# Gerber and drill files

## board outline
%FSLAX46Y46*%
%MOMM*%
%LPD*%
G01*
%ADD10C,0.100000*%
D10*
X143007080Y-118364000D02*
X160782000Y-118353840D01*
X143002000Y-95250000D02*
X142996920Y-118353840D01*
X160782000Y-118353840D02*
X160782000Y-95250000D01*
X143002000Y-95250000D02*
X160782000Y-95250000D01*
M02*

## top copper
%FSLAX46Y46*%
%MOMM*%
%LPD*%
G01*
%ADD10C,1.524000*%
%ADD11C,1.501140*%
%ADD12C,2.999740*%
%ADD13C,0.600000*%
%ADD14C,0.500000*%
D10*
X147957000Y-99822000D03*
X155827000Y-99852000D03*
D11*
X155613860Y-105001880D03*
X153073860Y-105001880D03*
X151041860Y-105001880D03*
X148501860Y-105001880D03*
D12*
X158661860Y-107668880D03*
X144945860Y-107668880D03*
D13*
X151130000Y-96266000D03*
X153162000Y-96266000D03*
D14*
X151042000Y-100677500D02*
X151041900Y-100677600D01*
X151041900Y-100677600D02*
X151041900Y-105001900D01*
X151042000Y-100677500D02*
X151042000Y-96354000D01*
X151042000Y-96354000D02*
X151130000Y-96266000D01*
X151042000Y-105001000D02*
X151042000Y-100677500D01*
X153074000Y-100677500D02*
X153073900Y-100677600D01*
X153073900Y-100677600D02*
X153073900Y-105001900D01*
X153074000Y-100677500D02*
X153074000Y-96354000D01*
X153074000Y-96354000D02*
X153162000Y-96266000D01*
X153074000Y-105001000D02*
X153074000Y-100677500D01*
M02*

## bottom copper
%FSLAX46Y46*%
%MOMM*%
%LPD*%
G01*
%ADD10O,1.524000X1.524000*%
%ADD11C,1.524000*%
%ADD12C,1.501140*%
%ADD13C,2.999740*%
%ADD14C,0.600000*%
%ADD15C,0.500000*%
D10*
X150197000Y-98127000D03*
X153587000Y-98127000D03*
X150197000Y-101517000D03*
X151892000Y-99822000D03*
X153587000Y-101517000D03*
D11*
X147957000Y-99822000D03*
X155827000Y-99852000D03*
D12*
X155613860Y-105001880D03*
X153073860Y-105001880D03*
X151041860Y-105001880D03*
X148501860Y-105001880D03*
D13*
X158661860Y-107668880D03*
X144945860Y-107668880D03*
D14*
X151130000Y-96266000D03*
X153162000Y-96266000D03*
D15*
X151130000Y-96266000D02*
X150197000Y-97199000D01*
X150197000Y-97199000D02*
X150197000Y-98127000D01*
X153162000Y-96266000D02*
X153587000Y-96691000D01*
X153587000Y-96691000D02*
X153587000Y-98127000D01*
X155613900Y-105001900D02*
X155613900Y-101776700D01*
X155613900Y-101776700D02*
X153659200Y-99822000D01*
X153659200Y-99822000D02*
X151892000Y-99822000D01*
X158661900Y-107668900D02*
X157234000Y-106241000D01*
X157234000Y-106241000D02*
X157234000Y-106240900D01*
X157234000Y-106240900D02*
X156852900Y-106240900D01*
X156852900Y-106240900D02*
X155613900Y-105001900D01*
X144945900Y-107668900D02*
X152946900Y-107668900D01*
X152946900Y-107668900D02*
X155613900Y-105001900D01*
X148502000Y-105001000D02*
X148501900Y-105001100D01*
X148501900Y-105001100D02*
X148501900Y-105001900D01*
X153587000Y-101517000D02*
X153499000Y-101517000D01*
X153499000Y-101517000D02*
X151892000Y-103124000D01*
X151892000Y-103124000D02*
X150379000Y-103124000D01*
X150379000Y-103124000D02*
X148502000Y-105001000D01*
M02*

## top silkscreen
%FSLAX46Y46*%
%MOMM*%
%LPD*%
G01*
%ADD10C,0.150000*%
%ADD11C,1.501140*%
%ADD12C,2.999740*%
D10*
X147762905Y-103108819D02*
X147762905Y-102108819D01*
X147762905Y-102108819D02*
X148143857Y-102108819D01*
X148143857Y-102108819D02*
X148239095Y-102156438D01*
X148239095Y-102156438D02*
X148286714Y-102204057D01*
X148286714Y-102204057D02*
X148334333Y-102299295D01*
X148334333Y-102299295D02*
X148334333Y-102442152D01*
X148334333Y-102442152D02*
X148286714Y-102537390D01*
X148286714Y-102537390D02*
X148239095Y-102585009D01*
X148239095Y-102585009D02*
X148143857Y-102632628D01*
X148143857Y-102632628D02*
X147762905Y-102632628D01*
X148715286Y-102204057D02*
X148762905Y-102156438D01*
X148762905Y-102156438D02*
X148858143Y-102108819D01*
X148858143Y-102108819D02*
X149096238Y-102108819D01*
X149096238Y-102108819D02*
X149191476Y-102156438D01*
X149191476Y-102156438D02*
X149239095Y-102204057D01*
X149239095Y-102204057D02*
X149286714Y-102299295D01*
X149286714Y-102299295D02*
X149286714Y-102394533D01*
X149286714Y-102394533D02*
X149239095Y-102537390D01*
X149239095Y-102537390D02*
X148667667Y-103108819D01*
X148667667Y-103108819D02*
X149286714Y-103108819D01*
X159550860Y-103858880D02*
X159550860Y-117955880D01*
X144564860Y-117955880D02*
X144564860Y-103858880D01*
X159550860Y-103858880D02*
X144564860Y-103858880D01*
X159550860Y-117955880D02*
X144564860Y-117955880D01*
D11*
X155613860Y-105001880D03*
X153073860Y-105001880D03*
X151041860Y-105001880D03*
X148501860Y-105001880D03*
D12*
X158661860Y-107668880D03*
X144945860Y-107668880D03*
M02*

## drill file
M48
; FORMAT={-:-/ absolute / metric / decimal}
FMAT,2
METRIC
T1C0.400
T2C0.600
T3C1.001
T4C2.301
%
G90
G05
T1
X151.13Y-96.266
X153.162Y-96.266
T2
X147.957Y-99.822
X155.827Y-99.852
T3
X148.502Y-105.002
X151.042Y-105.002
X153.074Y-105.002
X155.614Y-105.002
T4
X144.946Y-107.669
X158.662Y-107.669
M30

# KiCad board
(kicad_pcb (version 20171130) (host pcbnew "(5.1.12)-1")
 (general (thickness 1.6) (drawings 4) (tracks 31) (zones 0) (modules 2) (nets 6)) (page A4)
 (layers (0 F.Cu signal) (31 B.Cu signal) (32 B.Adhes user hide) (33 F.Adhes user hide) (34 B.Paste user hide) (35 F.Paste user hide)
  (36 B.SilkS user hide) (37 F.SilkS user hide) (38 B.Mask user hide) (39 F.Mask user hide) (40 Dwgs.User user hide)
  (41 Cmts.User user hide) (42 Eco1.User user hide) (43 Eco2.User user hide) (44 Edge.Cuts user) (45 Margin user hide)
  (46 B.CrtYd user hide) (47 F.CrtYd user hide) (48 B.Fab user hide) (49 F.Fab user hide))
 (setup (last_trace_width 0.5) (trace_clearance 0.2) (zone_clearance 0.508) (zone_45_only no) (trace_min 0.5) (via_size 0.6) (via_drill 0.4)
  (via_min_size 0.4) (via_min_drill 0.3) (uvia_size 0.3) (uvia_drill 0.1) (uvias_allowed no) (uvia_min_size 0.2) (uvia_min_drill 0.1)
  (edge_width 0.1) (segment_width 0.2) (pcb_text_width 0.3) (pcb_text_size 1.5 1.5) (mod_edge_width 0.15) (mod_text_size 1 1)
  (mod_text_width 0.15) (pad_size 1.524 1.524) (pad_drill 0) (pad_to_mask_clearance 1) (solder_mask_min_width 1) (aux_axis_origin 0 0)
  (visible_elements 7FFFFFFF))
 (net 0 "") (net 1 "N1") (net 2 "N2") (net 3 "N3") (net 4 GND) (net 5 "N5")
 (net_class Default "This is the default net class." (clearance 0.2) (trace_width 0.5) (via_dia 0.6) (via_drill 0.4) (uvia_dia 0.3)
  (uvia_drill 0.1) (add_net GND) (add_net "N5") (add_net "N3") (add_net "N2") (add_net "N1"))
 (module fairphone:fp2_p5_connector (layer B.Cu) (at 151.892 99.822)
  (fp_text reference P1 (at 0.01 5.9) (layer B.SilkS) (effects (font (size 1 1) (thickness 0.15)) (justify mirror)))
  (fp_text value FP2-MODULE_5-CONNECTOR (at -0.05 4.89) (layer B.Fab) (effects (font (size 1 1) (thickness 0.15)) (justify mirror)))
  (pad 5 smd oval (at -1.695 -1.695) (size 1.524 1.524) (layers B.Cu B.Paste B.Mask) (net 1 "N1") (solder_mask_margin 1))
  (pad 4 smd oval (at 1.695 -1.695) (size 1.524 1.524) (layers B.Cu B.Paste) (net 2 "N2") (solder_mask_margin 1))
  (pad 2 smd oval (at -1.695 1.695) (size 1.524 1.524) (layers B.Cu B.Paste B.Mask) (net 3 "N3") (solder_mask_margin 1))
  (pad 3 smd oval (at 0 0) (size 1.524 1.524) (layers B.Cu B.Paste B.Mask) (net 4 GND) (solder_mask_margin 1))
  (pad 1 smd oval (at 1.695 1.695) (size 1.524 1.524) (layers B.Cu B.Paste B.Mask) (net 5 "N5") (solder_mask_margin 1))
  (pad "" thru_hole circle (at -3.935 0) (size 1.524 1.524) (drill 0.6) (layers *.Cu *.Mask B.SilkS))
  (pad "" thru_hole circle (at 3.935 0.03) (size 1.524 1.524) (drill 0.6) (layers *.Cu *.Mask B.SilkS)))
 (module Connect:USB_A (layer F.Cu) (at 148.501 105.004)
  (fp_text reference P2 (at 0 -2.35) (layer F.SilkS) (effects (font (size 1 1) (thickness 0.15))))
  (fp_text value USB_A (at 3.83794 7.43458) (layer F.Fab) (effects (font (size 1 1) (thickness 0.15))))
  (fp_line (start 11.04986 -1.14512) (end 11.04986 12.95188) (layer F.SilkS) (width 0.15))
  (fp_line (start -3.93614 12.95188) (end -3.93614 -1.14512) (layer F.SilkS) (width 0.15))
  (fp_line (start 11.04986 -1.14512) (end -3.93614 -1.14512) (layer F.SilkS) (width 0.15))
  (fp_line (start 11.04986 12.95188) (end -3.93614 12.95188) (layer F.SilkS) (width 0.15))
  (pad 4 thru_hole circle (at 7.11286 -0.00212 270) (size 1.50114 1.50114) (drill 1.00076) (layers *.Cu *.Mask F.SilkS) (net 4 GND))
  (pad 3 thru_hole circle (at 4.57286 -0.00212 270) (size 1.50114 1.50114) (drill 1.00076) (layers *.Cu *.Mask F.SilkS) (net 2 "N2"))
  (pad 2 thru_hole circle (at 2.54086 -0.00212 270) (size 1.50114 1.50114) (drill 1.00076) (layers *.Cu *.Mask F.SilkS) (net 1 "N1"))
  (pad 1 thru_hole circle (at 0.00086 -0.00212 270) (size 1.50114 1.50114) (drill 1.00076) (layers *.Cu *.Mask F.SilkS) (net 5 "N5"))
  (pad 5 thru_hole circle (at 10.16086 2.66488 270) (size 2.99974 2.99974) (drill 2.30124) (layers *.Cu *.Mask F.SilkS) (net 4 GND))
  (pad 5 thru_hole circle (at -3.55514 2.66488 270) (size 2.99974 2.99974) (drill 2.30124) (layers *.Cu *.Mask F.SilkS) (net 4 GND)))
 (gr_line (start 143.00708 118.364) (end 160.782 118.35384) (layer Edge.Cuts) (width 0.1))
 (gr_line (start 143.002 95.25) (end 142.99692 118.35384) (angle 90) (layer Edge.Cuts) (width 0.1))
 (gr_line (start 160.782 118.35384) (end 160.782 95.25) (angle 90) (layer Edge.Cuts) (width 0.1))
 (gr_line (start 143.002 95.25) (end 160.782 95.25) (angle 90) (layer Edge.Cuts) (width 0.1))
 (segment (start 151.042 100.6775) (end 151.0419 100.6776) (width 0.5) (layer F.Cu) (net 1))
 (segment (start 151.0419 100.6776) (end 151.0419 105.0019) (width 0.5) (layer F.Cu) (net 1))
 (segment (start 151.042 100.6775) (end 151.042 96.354) (width 0.5) (layer F.Cu) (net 1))
 (segment (start 151.042 96.354) (end 151.13 96.266) (width 0.5) (layer F.Cu) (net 1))
 (segment (start 151.042 105.001) (end 151.042 100.6775) (width 0.5) (layer F.Cu) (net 1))
 (segment (start 151.13 96.266) (end 150.197 97.199) (width 0.5) (layer B.Cu) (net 1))
 (segment (start 150.197 97.199) (end 150.197 98.127) (width 0.5) (layer B.Cu) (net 1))
 (via (at 151.13 96.266) (size 0.6) (layers F.Cu B.Cu) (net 1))
 (segment (start 153.074 100.6775) (end 153.0739 100.6776) (width 0.5) (layer F.Cu) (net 2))
 (segment (start 153.0739 100.6776) (end 153.0739 105.0019) (width 0.5) (layer F.Cu) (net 2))
 (segment (start 153.074 100.6775) (end 153.074 96.354) (width 0.5) (layer F.Cu) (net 2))
 (segment (start 153.074 96.354) (end 153.162 96.266) (width 0.5) (layer F.Cu) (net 2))
 (segment (start 153.074 105.001) (end 153.074 100.6775) (width 0.5) (layer F.Cu) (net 2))
 (segment (start 153.162 96.266) (end 153.587 96.691) (width 0.5) (layer B.Cu) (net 2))
 (segment (start 153.587 96.691) (end 153.587 98.127) (width 0.5) (layer B.Cu) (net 2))
 (via (at 153.162 96.266) (size 0.6) (layers F.Cu B.Cu) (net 2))
 (segment (start 155.6139 105.0019) (end 155.6139 101.7767) (width 0.5) (layer B.Cu) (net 4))
 (segment (start 155.6139 101.7767) (end 153.6592 99.822) (width 0.5) (layer B.Cu) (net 4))
 (segment (start 153.6592 99.822) (end 151.892 99.822) (width 0.5) (layer B.Cu) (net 4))
 (segment (start 158.6619 107.6689) (end 157.234 106.241) (width 0.5) (layer B.Cu) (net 4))
 (segment (start 157.234 106.241) (end 157.234 106.2409) (width 0.5) (layer B.Cu) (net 4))
 (segment (start 157.234 106.2409) (end 156.8529 106.2409) (width 0.5) (layer B.Cu) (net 4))
 (segment (start 156.8529 106.2409) (end 155.6139 105.0019) (width 0.5) (layer B.Cu) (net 4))
 (segment (start 144.9459 107.6689) (end 152.9469 107.6689) (width 0.5) (layer B.Cu) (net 4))
 (segment (start 152.9469 107.6689) (end 155.6139 105.0019) (width 0.5) (layer B.Cu) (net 4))
 (segment (start 148.502 105.001) (end 148.5019 105.0011) (width 0.5) (layer B.Cu) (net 5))
 (segment (start 148.5019 105.0011) (end 148.5019 105.0019) (width 0.5) (layer B.Cu) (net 5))
 (segment (start 153.587 101.517) (end 153.499 101.517) (width 0.5) (layer B.Cu) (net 5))
 (segment (start 153.499 101.517) (end 151.892 103.124) (width 0.5) (layer B.Cu) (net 5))
 (segment (start 151.892 103.124) (end 150.379 103.124) (width 0.5) (layer B.Cu) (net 5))
 (segment (start 150.379 103.124) (end 148.502 105.001) (width 0.5) (layer B.Cu) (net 5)))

